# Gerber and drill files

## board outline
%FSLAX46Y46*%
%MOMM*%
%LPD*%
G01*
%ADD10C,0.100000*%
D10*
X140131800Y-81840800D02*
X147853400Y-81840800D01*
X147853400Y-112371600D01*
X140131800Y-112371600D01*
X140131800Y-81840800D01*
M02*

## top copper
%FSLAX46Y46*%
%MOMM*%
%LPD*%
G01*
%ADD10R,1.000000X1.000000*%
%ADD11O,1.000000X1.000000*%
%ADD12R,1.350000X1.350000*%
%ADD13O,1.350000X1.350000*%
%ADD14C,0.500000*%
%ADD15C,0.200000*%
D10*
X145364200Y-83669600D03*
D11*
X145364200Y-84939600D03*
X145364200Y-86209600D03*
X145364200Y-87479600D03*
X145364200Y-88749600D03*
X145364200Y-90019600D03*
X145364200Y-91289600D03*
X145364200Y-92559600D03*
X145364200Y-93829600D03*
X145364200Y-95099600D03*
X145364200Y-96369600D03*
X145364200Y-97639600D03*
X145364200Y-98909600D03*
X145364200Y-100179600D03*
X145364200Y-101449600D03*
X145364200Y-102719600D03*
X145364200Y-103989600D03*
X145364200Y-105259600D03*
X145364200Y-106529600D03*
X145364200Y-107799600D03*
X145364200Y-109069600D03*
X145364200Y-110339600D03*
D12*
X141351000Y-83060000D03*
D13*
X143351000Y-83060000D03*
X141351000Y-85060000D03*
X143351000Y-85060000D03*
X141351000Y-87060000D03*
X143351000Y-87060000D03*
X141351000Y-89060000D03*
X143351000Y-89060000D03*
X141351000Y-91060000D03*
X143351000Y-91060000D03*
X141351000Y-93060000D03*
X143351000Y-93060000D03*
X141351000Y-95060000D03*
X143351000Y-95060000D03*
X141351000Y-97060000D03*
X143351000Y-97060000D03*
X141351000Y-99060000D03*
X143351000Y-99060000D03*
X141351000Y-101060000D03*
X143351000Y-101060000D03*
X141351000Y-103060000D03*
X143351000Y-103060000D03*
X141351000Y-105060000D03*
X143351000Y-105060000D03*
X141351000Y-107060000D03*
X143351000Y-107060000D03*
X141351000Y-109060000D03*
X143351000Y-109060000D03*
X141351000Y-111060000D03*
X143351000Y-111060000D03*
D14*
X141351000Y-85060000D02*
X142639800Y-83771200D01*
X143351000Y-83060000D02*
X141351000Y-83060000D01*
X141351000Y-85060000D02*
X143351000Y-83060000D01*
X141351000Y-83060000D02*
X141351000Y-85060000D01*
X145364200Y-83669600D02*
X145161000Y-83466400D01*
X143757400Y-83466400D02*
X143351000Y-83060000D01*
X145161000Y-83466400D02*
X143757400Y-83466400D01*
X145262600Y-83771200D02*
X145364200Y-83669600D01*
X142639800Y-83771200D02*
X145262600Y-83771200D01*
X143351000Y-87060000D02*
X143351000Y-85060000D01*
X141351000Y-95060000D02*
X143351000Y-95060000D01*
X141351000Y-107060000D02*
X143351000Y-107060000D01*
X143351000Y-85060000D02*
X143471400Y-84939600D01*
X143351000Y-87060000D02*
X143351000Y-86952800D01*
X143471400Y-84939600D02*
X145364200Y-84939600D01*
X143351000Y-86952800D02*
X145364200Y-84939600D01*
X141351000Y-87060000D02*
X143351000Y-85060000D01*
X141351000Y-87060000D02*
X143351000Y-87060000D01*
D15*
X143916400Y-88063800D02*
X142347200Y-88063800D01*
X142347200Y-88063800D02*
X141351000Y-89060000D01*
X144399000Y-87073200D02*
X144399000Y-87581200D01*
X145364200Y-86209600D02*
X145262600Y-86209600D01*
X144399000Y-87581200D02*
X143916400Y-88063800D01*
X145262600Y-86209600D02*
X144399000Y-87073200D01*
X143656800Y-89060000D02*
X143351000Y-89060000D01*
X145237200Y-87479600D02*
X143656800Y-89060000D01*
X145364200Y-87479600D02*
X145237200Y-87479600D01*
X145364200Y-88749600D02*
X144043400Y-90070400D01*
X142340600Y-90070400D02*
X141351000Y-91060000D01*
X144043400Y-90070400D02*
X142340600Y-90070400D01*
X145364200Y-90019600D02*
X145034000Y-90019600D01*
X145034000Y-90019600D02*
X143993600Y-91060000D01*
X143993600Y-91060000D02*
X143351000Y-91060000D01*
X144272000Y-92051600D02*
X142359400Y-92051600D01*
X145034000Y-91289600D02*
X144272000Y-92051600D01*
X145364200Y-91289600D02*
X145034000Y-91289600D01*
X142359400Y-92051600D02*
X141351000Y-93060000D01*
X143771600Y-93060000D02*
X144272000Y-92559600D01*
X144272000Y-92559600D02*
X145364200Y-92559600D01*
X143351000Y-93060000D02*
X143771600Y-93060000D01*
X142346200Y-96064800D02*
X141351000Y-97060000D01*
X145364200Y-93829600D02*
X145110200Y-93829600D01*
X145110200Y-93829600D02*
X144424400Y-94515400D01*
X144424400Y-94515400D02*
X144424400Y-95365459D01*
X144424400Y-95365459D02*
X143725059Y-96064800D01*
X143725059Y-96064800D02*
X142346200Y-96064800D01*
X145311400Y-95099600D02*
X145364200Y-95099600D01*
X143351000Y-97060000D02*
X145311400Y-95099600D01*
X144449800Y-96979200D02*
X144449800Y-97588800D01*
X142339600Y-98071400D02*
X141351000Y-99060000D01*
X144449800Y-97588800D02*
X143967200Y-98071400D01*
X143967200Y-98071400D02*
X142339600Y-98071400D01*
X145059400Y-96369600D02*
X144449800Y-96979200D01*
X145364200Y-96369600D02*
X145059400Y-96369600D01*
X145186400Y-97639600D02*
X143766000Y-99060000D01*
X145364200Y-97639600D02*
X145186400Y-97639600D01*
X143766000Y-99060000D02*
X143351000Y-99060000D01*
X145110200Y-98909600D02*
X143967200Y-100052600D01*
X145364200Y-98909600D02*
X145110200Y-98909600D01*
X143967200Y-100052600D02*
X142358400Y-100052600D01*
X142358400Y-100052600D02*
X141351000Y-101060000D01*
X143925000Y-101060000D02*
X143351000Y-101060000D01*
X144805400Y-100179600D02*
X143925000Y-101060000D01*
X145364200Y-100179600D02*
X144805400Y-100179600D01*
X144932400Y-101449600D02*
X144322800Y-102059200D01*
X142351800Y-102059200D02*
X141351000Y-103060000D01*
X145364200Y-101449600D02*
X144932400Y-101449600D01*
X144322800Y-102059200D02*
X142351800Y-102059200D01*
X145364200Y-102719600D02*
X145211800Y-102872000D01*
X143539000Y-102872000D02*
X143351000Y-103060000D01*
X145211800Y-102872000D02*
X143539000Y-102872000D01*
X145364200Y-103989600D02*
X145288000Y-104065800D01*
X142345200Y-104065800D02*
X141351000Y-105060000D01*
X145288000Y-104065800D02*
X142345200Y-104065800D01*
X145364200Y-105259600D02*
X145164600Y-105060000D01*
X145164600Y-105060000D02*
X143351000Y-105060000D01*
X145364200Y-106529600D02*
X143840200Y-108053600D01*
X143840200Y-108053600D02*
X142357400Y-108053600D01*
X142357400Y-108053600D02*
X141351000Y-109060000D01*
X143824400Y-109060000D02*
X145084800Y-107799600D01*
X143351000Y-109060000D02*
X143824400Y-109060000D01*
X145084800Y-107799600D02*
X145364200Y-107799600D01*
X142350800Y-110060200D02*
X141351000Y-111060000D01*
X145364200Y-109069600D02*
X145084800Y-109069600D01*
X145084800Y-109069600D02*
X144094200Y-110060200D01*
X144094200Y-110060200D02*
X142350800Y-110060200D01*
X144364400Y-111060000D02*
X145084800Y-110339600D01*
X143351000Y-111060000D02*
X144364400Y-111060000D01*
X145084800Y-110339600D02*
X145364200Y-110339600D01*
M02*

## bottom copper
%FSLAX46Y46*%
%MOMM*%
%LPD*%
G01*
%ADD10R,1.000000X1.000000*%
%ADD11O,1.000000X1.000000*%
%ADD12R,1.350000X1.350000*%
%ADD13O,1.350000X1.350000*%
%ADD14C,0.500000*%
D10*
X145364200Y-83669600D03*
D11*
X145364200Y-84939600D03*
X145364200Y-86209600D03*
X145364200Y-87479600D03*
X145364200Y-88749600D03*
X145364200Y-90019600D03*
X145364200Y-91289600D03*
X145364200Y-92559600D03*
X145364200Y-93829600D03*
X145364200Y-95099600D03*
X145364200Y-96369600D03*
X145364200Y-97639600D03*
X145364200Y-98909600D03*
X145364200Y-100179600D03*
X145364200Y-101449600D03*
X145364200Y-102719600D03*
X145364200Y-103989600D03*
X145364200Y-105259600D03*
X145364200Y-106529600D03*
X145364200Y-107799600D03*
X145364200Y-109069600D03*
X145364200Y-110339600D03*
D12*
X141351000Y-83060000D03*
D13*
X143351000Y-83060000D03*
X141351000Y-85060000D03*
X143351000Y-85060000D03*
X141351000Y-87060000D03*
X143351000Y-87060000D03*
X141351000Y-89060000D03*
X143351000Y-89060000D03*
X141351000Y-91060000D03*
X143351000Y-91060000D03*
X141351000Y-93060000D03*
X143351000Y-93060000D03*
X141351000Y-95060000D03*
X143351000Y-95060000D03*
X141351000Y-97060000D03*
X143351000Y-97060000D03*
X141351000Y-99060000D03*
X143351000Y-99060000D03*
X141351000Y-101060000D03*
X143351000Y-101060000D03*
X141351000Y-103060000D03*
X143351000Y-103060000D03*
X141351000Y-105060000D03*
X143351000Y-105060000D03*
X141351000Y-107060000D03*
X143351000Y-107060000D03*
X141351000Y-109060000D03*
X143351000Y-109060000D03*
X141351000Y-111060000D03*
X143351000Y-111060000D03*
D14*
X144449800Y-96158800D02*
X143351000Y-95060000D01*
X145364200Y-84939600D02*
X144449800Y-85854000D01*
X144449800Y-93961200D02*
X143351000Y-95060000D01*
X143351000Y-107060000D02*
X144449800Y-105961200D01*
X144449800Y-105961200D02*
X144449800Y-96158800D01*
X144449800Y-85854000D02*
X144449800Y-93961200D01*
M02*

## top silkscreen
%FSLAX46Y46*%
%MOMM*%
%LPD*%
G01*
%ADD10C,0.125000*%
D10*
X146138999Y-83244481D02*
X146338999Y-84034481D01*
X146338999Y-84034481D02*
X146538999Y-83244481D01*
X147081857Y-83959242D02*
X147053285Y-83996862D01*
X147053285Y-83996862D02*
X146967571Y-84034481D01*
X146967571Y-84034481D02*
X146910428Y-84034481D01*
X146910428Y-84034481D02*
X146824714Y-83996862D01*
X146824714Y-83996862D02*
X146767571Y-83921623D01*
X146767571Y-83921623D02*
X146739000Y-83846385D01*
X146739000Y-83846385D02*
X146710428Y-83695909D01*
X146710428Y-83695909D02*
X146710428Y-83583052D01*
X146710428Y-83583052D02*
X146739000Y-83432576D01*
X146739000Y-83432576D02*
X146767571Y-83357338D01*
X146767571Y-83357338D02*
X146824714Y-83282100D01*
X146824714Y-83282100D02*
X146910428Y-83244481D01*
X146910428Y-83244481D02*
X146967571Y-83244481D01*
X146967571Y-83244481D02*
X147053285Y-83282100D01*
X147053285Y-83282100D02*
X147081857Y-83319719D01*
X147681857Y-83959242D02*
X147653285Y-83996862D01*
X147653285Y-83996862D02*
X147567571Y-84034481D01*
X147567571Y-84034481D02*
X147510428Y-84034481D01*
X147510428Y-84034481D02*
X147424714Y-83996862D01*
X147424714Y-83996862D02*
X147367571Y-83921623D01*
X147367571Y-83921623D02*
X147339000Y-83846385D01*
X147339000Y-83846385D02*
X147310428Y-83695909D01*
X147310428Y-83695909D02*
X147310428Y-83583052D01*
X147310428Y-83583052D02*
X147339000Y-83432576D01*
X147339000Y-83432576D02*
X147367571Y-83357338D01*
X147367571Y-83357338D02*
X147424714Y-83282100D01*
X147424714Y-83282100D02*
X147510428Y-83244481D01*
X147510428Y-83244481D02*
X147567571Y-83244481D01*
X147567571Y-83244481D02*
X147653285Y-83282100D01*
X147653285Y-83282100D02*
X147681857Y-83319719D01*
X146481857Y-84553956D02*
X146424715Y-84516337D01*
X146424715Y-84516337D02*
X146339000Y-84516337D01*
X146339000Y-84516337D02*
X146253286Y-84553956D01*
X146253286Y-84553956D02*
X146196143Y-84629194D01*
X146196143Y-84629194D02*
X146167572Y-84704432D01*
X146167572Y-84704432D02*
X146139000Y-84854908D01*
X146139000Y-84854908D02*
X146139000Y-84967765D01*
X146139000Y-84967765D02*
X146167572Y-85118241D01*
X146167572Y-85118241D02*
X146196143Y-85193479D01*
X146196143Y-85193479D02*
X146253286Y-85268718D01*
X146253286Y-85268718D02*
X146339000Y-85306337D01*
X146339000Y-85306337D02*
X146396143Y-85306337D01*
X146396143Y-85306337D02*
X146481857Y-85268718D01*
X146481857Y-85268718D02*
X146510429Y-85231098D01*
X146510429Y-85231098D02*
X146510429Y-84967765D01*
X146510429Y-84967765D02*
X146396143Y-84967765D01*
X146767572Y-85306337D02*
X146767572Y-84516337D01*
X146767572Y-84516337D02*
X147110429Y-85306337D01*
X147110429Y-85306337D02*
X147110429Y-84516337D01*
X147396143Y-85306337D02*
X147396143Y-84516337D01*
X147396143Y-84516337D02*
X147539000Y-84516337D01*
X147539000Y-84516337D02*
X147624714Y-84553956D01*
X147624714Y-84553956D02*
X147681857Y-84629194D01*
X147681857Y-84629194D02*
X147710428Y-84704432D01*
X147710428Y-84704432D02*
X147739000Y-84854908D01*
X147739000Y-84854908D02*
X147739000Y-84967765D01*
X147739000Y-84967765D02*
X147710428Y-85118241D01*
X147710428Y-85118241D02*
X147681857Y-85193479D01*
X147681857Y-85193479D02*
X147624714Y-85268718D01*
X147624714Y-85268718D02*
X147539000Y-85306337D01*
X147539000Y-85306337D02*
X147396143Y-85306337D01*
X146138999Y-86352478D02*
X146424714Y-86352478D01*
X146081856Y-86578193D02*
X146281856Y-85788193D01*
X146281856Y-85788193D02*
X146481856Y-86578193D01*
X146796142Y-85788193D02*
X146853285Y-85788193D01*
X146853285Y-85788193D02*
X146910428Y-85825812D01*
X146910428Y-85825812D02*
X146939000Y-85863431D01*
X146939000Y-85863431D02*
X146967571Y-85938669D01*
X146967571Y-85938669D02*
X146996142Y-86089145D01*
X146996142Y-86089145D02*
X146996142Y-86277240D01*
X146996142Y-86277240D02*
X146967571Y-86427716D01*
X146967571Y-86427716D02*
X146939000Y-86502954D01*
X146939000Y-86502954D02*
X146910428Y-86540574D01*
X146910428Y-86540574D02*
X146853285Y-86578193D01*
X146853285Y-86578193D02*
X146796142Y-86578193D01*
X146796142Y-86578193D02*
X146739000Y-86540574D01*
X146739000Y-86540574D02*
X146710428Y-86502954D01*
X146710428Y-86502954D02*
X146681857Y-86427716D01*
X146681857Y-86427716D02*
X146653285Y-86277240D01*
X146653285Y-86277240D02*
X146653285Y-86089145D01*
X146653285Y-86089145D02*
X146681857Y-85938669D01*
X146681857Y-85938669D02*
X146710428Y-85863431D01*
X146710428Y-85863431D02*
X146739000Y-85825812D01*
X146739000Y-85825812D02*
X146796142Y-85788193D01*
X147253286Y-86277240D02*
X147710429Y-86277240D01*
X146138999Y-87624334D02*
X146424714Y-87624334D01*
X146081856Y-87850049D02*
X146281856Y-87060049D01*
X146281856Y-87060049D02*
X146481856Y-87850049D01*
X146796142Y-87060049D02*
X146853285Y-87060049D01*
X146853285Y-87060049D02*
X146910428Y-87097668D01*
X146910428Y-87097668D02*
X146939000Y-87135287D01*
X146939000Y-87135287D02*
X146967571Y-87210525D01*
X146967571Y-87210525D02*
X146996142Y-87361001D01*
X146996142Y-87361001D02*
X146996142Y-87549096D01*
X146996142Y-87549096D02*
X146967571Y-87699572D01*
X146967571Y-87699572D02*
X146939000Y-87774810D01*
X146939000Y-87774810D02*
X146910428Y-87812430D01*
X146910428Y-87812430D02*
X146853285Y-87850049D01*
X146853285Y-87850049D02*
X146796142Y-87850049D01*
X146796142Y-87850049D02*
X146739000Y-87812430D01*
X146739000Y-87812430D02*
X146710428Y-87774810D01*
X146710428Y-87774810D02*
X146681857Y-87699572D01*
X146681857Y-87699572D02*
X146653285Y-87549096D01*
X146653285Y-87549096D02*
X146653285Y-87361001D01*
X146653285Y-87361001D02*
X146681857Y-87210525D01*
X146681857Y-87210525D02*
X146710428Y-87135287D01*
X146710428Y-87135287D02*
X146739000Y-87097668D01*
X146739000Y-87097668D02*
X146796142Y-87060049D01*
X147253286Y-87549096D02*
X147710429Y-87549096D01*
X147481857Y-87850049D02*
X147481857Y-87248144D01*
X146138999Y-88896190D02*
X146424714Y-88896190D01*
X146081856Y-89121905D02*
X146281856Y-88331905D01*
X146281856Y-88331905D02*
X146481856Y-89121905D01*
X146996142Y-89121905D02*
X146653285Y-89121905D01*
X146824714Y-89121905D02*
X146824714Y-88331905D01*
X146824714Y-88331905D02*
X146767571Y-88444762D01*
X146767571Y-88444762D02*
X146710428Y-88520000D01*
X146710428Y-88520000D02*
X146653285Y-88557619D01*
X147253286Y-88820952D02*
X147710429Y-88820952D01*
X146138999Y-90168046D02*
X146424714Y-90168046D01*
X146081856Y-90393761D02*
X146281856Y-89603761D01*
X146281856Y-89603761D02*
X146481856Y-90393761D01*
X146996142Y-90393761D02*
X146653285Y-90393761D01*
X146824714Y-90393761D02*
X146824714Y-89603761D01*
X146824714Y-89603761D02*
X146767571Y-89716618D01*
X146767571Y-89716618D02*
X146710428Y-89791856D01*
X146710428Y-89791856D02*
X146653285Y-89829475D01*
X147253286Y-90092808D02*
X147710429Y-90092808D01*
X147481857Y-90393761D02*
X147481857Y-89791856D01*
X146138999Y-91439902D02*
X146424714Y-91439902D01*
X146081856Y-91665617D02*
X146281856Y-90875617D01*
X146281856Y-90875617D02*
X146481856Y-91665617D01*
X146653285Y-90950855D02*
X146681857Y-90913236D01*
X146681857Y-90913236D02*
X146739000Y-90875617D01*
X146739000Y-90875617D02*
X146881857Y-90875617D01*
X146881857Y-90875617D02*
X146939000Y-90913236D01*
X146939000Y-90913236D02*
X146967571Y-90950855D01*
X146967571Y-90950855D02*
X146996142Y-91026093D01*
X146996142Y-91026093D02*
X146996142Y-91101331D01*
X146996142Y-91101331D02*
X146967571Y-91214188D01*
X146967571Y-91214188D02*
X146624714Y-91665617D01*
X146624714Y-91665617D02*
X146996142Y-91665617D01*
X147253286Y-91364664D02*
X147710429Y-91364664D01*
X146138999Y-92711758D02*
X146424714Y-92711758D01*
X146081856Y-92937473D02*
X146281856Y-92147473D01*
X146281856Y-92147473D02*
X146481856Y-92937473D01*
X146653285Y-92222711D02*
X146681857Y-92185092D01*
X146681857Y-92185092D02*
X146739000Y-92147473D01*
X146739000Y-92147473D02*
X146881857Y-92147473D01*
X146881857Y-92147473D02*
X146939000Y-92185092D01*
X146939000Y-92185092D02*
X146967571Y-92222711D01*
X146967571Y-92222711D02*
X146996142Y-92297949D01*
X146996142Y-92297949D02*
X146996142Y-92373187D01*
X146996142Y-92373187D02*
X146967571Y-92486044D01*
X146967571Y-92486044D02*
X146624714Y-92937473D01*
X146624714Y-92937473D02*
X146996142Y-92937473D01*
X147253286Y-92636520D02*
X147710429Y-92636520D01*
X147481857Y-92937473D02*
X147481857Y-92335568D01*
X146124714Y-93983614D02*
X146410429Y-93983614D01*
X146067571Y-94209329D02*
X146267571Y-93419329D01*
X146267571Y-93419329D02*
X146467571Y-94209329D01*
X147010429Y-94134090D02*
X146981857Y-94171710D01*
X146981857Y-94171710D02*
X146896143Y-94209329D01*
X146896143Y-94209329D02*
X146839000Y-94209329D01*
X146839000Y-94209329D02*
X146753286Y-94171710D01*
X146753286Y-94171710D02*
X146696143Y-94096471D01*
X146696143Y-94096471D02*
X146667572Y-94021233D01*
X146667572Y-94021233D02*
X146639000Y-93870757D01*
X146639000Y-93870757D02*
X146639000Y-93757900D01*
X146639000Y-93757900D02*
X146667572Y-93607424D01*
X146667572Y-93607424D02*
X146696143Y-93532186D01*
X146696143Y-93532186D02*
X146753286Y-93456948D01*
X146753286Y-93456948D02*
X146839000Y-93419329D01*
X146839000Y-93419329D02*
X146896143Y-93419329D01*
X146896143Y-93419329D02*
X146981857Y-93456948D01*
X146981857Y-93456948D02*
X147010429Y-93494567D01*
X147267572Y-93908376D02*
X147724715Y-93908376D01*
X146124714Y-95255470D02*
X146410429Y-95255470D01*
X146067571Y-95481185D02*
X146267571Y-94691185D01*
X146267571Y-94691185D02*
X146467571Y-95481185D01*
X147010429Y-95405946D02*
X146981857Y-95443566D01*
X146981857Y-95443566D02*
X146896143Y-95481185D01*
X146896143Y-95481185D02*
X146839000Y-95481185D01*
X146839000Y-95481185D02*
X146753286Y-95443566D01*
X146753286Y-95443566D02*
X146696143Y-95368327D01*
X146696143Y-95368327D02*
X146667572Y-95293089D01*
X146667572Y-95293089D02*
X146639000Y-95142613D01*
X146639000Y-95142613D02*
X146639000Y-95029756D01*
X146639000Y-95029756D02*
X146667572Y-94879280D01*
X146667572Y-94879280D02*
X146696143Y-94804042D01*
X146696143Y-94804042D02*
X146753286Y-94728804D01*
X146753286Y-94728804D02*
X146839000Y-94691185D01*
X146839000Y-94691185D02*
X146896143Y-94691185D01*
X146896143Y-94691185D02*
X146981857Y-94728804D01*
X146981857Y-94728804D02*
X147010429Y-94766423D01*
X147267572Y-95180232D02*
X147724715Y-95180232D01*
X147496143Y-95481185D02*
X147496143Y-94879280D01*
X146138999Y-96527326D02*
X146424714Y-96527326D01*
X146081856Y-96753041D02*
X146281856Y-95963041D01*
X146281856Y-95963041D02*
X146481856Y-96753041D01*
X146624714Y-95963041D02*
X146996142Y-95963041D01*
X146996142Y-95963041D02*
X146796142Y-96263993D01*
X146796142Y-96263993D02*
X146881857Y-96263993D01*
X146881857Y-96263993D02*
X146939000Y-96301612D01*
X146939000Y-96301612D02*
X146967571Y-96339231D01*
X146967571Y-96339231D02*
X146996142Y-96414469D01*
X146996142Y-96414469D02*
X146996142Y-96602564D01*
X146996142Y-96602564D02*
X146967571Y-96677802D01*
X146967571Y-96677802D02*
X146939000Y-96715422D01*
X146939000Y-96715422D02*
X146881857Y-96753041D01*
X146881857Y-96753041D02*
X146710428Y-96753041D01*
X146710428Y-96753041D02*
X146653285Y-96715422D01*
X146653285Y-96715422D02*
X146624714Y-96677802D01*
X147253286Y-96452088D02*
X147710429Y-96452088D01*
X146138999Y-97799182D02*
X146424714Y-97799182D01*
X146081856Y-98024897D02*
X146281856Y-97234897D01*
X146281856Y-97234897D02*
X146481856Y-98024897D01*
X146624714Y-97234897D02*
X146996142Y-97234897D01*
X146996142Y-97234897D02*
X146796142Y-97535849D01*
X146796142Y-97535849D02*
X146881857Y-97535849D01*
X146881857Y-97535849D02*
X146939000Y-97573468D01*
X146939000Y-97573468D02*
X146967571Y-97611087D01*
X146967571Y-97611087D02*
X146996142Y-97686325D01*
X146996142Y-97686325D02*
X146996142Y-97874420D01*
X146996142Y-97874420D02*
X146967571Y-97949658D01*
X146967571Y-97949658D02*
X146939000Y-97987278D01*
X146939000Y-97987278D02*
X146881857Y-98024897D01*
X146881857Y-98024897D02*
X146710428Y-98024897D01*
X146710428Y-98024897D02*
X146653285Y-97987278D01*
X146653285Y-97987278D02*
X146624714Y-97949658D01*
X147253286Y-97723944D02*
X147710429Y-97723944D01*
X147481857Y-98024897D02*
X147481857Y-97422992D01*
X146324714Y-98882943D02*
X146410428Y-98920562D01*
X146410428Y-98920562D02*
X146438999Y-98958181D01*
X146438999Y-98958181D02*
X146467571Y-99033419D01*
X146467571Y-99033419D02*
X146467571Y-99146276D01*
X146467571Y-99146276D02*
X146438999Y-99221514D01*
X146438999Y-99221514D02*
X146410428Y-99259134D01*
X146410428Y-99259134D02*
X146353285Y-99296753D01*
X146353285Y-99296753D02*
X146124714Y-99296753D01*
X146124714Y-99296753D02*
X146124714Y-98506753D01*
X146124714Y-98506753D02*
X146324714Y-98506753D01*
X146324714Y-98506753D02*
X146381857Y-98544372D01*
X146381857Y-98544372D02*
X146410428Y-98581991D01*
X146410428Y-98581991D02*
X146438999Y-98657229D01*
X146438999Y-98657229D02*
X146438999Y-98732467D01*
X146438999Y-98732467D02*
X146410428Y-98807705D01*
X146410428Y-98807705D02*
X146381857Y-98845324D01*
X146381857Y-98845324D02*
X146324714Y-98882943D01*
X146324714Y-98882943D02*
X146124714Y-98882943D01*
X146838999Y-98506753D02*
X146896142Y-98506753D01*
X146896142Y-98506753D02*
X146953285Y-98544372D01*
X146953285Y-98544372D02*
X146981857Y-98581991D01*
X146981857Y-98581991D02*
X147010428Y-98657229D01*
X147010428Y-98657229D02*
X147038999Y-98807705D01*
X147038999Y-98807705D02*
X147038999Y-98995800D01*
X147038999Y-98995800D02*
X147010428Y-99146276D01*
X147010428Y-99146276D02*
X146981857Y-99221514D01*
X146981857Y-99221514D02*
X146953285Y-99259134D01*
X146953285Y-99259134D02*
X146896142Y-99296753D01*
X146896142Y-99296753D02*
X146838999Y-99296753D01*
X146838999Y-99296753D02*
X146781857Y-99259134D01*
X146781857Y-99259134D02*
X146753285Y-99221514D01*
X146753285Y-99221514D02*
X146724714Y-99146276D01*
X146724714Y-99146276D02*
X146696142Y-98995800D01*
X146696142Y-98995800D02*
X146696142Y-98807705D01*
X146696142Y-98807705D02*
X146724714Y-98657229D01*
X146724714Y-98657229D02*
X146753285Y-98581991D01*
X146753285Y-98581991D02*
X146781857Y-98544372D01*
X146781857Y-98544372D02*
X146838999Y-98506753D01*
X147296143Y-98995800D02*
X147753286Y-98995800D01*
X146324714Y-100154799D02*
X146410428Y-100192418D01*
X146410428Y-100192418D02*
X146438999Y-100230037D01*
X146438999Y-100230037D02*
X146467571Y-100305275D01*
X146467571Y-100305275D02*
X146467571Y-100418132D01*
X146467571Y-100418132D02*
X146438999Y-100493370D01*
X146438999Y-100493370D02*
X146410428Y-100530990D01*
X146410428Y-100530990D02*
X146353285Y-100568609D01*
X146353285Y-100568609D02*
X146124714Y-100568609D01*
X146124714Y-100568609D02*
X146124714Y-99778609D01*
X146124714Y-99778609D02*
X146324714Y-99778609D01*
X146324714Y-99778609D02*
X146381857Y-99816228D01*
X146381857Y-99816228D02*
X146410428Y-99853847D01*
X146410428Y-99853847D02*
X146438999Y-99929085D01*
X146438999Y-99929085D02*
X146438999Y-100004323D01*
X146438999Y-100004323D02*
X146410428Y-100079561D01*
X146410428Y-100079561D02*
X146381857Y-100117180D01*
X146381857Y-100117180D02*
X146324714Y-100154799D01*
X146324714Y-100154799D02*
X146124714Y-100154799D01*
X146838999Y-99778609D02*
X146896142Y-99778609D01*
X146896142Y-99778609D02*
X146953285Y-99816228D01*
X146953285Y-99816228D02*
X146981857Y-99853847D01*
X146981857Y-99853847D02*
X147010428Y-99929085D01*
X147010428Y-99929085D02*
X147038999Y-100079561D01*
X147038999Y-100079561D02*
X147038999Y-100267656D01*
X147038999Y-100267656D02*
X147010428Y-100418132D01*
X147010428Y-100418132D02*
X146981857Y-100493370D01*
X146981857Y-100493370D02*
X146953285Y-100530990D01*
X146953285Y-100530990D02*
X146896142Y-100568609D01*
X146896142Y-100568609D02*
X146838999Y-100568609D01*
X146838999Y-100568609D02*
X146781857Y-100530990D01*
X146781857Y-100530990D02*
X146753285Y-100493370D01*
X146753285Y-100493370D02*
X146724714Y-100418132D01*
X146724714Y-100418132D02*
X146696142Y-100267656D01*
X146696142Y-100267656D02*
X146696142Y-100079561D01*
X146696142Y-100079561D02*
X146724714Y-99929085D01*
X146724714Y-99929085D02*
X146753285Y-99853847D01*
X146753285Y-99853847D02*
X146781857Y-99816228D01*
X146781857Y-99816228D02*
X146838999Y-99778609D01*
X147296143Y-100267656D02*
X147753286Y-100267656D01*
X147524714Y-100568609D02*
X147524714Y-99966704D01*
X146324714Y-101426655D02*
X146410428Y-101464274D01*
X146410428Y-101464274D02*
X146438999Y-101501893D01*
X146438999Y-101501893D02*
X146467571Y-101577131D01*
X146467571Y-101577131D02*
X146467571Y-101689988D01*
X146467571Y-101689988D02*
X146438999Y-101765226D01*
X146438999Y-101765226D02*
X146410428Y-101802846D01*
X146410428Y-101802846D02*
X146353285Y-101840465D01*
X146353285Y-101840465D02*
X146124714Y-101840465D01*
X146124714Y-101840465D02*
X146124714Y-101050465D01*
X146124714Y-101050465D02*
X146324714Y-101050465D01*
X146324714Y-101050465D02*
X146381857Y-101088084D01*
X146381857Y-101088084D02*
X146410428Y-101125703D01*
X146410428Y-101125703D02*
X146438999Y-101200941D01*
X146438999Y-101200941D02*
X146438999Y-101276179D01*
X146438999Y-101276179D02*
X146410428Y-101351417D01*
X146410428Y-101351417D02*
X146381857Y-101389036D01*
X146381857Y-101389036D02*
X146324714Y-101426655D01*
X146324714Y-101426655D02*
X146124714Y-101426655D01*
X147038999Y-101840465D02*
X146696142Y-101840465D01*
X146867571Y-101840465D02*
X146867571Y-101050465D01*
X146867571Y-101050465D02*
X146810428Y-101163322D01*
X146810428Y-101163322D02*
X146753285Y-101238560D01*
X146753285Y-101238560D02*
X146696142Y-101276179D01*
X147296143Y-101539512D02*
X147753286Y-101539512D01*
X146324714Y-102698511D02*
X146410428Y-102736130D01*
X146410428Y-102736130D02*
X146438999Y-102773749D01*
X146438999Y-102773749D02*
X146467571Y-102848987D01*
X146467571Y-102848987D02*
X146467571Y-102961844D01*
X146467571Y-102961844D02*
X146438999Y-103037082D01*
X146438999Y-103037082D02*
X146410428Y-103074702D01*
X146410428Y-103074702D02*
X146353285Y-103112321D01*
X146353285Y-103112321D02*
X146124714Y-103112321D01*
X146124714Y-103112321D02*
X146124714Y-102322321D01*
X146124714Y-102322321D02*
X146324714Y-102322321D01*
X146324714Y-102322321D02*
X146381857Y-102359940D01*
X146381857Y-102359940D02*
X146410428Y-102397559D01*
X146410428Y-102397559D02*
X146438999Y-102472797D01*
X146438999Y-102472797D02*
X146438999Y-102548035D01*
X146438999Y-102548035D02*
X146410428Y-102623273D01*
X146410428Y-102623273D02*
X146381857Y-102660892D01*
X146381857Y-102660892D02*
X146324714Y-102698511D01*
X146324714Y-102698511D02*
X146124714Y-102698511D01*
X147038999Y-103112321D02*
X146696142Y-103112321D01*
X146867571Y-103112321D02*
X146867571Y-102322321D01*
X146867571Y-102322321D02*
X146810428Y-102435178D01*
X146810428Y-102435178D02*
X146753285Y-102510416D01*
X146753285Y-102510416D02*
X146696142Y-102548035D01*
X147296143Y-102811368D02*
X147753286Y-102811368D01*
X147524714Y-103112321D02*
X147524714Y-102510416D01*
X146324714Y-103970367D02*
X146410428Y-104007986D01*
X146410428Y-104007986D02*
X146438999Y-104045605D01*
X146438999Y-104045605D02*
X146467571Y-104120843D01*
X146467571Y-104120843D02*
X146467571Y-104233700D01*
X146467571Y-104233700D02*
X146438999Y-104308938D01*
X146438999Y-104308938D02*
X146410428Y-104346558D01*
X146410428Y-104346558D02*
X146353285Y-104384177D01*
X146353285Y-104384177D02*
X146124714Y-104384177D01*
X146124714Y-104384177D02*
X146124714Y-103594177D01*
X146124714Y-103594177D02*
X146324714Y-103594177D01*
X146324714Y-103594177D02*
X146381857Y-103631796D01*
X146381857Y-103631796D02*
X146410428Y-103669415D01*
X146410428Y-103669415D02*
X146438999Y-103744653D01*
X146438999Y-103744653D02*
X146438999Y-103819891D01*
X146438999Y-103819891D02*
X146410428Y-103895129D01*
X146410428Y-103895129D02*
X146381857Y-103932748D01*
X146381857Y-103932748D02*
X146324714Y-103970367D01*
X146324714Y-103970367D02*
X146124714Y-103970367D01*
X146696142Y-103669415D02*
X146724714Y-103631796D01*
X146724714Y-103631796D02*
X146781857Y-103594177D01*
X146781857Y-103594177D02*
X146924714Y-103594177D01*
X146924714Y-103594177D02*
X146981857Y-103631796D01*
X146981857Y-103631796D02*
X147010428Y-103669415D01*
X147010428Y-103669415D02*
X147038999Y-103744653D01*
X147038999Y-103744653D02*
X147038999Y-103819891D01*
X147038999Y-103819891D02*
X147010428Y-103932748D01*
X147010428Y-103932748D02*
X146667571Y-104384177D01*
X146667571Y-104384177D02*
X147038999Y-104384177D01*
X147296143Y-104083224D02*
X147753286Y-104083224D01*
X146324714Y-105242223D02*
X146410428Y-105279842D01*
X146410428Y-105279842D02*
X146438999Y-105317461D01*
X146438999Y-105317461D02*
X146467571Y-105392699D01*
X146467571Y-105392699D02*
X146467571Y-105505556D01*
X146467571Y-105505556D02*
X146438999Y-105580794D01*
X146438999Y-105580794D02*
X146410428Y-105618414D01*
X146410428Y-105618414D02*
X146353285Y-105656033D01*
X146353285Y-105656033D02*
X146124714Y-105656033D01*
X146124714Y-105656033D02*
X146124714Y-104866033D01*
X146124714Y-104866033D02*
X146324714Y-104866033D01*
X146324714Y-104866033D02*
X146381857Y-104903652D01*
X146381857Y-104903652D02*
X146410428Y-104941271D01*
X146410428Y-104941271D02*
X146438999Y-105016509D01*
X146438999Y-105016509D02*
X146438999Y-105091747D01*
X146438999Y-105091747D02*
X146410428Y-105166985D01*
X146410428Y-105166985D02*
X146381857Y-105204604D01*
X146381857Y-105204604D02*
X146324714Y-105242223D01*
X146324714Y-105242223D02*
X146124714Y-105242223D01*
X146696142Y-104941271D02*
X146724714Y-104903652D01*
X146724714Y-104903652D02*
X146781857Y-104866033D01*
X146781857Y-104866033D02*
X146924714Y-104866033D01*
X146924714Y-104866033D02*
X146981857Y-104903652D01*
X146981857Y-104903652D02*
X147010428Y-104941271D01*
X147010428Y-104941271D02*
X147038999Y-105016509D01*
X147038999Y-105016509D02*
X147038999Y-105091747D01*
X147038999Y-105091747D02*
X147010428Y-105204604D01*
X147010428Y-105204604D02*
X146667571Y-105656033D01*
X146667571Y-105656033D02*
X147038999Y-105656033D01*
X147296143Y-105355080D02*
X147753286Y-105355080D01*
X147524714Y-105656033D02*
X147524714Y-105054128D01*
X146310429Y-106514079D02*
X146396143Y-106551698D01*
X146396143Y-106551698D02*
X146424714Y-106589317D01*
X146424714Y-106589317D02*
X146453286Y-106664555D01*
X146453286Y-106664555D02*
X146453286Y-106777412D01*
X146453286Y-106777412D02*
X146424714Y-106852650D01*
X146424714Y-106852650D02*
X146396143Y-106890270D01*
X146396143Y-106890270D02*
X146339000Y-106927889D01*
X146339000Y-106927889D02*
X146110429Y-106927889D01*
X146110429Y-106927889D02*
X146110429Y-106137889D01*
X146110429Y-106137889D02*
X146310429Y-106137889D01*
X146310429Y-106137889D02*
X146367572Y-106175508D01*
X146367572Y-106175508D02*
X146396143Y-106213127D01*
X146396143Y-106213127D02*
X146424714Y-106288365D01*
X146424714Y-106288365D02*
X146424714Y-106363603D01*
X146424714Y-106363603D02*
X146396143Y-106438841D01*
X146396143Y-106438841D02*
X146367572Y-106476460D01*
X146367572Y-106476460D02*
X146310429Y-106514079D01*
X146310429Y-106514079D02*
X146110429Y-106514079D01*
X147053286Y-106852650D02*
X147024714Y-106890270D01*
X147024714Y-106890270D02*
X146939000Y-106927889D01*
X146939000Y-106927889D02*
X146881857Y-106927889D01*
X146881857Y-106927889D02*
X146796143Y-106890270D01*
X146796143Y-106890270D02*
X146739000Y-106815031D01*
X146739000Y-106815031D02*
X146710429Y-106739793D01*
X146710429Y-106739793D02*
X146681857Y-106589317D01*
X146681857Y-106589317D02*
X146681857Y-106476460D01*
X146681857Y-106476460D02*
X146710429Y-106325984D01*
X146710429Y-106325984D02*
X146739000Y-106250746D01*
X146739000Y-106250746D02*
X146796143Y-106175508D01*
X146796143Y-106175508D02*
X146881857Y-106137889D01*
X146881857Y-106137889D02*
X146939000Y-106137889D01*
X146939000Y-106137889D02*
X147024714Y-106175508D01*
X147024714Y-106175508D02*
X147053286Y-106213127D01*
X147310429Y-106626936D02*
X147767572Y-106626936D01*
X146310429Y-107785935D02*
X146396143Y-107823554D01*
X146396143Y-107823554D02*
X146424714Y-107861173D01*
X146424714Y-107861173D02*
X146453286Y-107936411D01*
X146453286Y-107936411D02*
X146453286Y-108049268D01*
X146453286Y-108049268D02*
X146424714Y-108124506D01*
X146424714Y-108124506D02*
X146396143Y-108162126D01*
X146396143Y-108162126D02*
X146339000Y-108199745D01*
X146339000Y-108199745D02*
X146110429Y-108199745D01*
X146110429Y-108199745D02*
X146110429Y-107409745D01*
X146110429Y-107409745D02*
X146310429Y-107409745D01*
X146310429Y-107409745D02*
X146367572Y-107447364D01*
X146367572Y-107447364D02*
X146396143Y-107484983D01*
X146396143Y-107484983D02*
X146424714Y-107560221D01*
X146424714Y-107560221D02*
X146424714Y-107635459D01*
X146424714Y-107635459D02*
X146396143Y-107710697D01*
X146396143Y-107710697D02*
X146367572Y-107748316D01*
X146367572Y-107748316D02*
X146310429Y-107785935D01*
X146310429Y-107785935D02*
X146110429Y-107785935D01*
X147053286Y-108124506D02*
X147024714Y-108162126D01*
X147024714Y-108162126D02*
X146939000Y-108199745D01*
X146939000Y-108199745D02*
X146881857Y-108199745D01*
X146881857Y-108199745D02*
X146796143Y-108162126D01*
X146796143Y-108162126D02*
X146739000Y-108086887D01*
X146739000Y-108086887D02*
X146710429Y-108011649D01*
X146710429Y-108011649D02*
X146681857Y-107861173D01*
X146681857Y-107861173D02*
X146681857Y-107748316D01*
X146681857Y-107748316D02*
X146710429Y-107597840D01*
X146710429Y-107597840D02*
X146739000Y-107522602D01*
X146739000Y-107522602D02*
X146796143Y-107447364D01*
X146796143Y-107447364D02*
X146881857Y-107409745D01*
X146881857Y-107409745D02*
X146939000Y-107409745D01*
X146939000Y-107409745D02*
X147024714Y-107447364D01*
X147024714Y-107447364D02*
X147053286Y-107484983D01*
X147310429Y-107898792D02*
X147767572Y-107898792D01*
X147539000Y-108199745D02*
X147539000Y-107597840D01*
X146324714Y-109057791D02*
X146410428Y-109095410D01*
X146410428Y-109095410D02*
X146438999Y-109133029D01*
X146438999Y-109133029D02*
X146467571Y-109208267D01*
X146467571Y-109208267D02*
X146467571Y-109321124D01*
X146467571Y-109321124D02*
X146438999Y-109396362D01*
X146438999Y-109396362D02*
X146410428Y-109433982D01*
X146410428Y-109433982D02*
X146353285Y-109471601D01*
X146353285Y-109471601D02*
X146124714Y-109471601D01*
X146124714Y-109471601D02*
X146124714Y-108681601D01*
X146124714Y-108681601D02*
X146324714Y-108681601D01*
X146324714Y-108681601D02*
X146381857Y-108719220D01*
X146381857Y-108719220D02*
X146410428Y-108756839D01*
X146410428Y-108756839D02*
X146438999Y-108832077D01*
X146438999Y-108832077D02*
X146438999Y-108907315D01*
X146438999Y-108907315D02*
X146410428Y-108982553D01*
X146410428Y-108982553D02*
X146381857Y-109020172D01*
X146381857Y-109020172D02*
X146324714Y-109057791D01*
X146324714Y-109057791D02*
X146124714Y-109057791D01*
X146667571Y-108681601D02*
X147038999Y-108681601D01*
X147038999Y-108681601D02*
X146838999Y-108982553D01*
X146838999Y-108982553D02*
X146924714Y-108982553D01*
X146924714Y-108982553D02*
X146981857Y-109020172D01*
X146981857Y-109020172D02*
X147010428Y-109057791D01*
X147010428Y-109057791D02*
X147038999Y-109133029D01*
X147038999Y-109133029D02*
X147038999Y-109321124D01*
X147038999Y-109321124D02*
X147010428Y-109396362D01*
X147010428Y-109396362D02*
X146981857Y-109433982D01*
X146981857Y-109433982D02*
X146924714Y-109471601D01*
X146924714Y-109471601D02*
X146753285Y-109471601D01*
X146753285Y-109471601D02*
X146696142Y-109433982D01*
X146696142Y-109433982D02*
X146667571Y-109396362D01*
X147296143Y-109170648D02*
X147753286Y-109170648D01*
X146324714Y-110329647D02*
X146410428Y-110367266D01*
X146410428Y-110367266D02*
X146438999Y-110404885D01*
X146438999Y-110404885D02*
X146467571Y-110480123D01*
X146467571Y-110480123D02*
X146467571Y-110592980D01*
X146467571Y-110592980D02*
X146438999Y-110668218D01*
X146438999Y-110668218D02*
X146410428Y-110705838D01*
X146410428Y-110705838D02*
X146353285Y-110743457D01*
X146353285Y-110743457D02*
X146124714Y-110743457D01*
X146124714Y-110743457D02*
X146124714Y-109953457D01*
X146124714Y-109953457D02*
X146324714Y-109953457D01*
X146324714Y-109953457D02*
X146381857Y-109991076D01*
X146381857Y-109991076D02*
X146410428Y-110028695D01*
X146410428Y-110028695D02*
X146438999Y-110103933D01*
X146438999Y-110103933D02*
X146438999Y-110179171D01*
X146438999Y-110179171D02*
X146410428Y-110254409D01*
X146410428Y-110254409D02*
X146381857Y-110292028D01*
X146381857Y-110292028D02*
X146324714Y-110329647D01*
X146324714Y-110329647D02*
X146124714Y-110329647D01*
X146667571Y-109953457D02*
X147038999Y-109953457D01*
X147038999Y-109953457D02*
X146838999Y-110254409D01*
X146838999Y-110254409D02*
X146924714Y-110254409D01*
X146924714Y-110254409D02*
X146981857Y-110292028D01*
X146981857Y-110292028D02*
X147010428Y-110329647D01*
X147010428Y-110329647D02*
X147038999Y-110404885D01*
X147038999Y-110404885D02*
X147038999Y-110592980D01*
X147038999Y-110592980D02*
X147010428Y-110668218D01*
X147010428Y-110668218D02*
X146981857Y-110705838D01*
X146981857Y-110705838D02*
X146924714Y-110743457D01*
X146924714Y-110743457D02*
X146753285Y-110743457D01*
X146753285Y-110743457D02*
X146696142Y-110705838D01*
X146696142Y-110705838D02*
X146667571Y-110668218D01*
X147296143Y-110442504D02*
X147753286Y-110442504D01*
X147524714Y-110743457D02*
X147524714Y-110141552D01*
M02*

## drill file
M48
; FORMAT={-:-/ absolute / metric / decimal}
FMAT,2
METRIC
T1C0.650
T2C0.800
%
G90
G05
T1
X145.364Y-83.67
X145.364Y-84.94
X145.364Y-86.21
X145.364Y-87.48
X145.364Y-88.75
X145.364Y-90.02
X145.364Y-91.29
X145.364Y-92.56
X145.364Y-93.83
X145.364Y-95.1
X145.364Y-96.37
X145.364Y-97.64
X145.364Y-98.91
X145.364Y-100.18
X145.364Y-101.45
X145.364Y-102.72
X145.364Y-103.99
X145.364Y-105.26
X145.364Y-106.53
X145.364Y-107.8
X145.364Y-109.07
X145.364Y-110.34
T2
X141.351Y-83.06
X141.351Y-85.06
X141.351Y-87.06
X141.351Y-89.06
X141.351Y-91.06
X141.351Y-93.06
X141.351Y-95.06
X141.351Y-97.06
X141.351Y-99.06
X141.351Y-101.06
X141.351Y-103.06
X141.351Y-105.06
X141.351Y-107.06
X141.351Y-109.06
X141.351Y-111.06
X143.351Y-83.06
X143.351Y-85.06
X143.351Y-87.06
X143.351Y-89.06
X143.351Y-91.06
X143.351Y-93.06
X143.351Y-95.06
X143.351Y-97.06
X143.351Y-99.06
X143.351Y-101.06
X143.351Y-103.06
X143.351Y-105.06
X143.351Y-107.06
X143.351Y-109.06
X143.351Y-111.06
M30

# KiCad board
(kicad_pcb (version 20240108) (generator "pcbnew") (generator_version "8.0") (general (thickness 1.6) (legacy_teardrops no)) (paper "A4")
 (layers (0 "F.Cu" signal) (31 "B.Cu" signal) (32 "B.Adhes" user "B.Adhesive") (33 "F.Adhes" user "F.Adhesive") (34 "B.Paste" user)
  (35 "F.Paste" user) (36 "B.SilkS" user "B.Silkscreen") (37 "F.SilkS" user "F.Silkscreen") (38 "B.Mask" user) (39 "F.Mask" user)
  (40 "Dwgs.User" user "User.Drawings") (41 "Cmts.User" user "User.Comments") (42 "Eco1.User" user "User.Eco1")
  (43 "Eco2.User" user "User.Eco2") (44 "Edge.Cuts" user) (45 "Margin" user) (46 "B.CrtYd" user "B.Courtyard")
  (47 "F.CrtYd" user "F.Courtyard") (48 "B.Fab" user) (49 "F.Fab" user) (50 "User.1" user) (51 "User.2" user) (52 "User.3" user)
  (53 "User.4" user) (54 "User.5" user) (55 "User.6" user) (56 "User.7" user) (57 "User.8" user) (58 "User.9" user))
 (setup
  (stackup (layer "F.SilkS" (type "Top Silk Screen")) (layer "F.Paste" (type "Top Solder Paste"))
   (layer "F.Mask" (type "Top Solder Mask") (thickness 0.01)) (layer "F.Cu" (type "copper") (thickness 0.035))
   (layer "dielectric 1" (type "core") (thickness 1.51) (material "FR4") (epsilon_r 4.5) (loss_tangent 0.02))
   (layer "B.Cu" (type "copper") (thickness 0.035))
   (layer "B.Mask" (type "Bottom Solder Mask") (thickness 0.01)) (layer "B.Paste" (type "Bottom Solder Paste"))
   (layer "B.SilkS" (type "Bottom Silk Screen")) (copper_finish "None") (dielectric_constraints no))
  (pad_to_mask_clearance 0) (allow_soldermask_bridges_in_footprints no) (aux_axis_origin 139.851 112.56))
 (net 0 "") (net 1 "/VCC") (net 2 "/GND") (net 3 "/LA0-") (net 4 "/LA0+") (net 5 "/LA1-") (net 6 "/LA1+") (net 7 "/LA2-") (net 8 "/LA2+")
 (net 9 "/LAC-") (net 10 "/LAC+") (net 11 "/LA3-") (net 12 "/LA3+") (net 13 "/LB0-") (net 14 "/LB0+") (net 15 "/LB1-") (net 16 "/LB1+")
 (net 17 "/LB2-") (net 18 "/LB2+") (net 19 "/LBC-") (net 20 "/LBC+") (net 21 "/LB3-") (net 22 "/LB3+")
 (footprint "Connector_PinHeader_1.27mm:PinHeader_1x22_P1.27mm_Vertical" (layer "B.Cu") (at 145.3642 83.6696 180)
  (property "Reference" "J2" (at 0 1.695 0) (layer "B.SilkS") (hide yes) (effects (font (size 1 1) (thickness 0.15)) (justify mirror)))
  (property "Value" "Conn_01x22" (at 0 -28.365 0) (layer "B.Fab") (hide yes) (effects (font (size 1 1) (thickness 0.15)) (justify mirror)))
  (pad "1" thru_hole rect (at 0 0 180) (size 1 1) (drill 0.65) (layers "*.Cu" "*.Mask") (remove_unused_layers no) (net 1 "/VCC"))
  (pad "2" thru_hole oval (at 0 -1.27 180) (size 1 1) (drill 0.65) (layers "*.Cu" "*.Mask") (remove_unused_layers no) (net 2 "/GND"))
  (pad "3" thru_hole oval (at 0 -2.54 180) (size 1 1) (drill 0.65) (layers "*.Cu" "*.Mask") (remove_unused_layers no) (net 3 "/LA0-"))
  (pad "4" thru_hole oval (at 0 -3.81 180) (size 1 1) (drill 0.65) (layers "*.Cu" "*.Mask") (remove_unused_layers no) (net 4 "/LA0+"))
  (pad "5" thru_hole oval (at 0 -5.08 180) (size 1 1) (drill 0.65) (layers "*.Cu" "*.Mask") (remove_unused_layers no) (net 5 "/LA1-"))
  (pad "6" thru_hole oval (at 0 -6.35 180) (size 1 1) (drill 0.65) (layers "*.Cu" "*.Mask") (remove_unused_layers no) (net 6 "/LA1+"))
  (pad "7" thru_hole oval (at 0 -7.62 180) (size 1 1) (drill 0.65) (layers "*.Cu" "*.Mask") (remove_unused_layers no) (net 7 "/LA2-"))
  (pad "8" thru_hole oval (at 0 -8.89 180) (size 1 1) (drill 0.65) (layers "*.Cu" "*.Mask") (remove_unused_layers no) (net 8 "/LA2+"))
  (pad "9" thru_hole oval (at 0 -10.16 180) (size 1 1) (drill 0.65) (layers "*.Cu" "*.Mask") (remove_unused_layers no) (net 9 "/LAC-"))
  (pad "10" thru_hole oval (at 0 -11.43 180) (size 1 1) (drill 0.65) (layers "*.Cu" "*.Mask") (remove_unused_layers no) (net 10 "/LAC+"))
  (pad "11" thru_hole oval (at 0 -12.7 180) (size 1 1) (drill 0.65) (layers "*.Cu" "*.Mask") (remove_unused_layers no) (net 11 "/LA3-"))
  (pad "12" thru_hole oval (at 0 -13.97 180) (size 1 1) (drill 0.65) (layers "*.Cu" "*.Mask") (remove_unused_layers no) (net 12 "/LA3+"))
  (pad "13" thru_hole oval (at 0 -15.24 180) (size 1 1) (drill 0.65) (layers "*.Cu" "*.Mask") (remove_unused_layers no) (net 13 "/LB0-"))
  (pad "14" thru_hole oval (at 0 -16.51 180) (size 1 1) (drill 0.65) (layers "*.Cu" "*.Mask") (remove_unused_layers no) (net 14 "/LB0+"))
  (pad "15" thru_hole oval (at 0 -17.78 180) (size 1 1) (drill 0.65) (layers "*.Cu" "*.Mask") (remove_unused_layers no) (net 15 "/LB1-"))
  (pad "16" thru_hole oval (at 0 -19.05 180) (size 1 1) (drill 0.65) (layers "*.Cu" "*.Mask") (remove_unused_layers no) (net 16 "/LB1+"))
  (pad "17" thru_hole oval (at 0 -20.32 180) (size 1 1) (drill 0.65) (layers "*.Cu" "*.Mask") (remove_unused_layers no) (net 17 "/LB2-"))
  (pad "18" thru_hole oval (at 0 -21.59 180) (size 1 1) (drill 0.65) (layers "*.Cu" "*.Mask") (remove_unused_layers no) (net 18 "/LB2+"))
  (pad "19" thru_hole oval (at 0 -22.86 180) (size 1 1) (drill 0.65) (layers "*.Cu" "*.Mask") (remove_unused_layers no) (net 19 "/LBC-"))
  (pad "20" thru_hole oval (at 0 -24.13 180) (size 1 1) (drill 0.65) (layers "*.Cu" "*.Mask") (remove_unused_layers no) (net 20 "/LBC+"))
  (pad "21" thru_hole oval (at 0 -25.4 180) (size 1 1) (drill 0.65) (layers "*.Cu" "*.Mask") (remove_unused_layers no) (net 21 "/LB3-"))
  (pad "22" thru_hole oval (at 0 -26.67 180) (size 1 1) (drill 0.65) (layers "*.Cu" "*.Mask") (remove_unused_layers no) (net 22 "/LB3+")))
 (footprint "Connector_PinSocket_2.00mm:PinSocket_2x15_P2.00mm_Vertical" (layer "B.Cu") (at 141.351 83.06 180)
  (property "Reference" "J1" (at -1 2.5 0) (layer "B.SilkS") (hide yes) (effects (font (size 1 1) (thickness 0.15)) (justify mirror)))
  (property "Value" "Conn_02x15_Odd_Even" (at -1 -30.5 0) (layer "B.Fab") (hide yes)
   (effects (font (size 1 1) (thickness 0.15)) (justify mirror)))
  (pad "1" thru_hole rect (at 0 0 180) (size 1.35 1.35) (drill 0.8) (layers "*.Cu" "*.Mask") (remove_unused_layers no) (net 1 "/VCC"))
  (pad "2" thru_hole oval (at -2 0 180) (size 1.35 1.35) (drill 0.8) (layers "*.Cu" "*.Mask") (remove_unused_layers no) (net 1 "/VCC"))
  (pad "3" thru_hole oval (at 0 -2 180) (size 1.35 1.35) (drill 0.8) (layers "*.Cu" "*.Mask") (remove_unused_layers no) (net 1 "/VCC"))
  (pad "4" thru_hole oval (at -2 -2 180) (size 1.35 1.35) (drill 0.8) (layers "*.Cu" "*.Mask") (remove_unused_layers no) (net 2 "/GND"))
  (pad "5" thru_hole oval (at 0 -4 180) (size 1.35 1.35) (drill 0.8) (layers "*.Cu" "*.Mask") (remove_unused_layers no) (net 2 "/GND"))
  (pad "6" thru_hole oval (at -2 -4 180) (size 1.35 1.35) (drill 0.8) (layers "*.Cu" "*.Mask") (remove_unused_layers no) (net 2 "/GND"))
  (pad "7" thru_hole oval (at 0 -6 180) (size 1.35 1.35) (drill 0.8) (layers "*.Cu" "*.Mask") (remove_unused_layers no) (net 3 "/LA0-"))
  (pad "8" thru_hole oval (at -2 -6 180) (size 1.35 1.35) (drill 0.8) (layers "*.Cu" "*.Mask") (remove_unused_layers no) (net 4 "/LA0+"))
  (pad "9" thru_hole oval (at 0 -8 180) (size 1.35 1.35) (drill 0.8) (layers "*.Cu" "*.Mask") (remove_unused_layers no) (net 5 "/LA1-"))
  (pad "10" thru_hole oval (at -2 -8 180) (size 1.35 1.35) (drill 0.8) (layers "*.Cu" "*.Mask") (remove_unused_layers no) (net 6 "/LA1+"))
  (pad "11" thru_hole oval (at 0 -10 180) (size 1.35 1.35) (drill 0.8) (layers "*.Cu" "*.Mask") (remove_unused_layers no) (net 7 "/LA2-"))
  (pad "12" thru_hole oval (at -2 -10 180) (size 1.35 1.35) (drill 0.8) (layers "*.Cu" "*.Mask") (remove_unused_layers no) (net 8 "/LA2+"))
  (pad "13" thru_hole oval (at 0 -12 180) (size 1.35 1.35) (drill 0.8) (layers "*.Cu" "*.Mask") (remove_unused_layers no) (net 2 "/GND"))
  (pad "14" thru_hole oval (at -2 -12 180) (size 1.35 1.35) (drill 0.8) (layers "*.Cu" "*.Mask") (remove_unused_layers no) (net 2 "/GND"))
  (pad "15" thru_hole oval (at 0 -14 180) (size 1.35 1.35) (drill 0.8) (layers "*.Cu" "*.Mask") (remove_unused_layers no) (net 9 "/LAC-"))
  (pad "16" thru_hole oval (at -2 -14 180) (size 1.35 1.35) (drill 0.8) (layers "*.Cu" "*.Mask") (remove_unused_layers no) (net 10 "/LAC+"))
  (pad "17" thru_hole oval (at 0 -16 180) (size 1.35 1.35) (drill 0.8) (layers "*.Cu" "*.Mask") (remove_unused_layers no) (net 11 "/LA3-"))
  (pad "18" thru_hole oval (at -2 -16 180) (size 1.35 1.35) (drill 0.8) (layers "*.Cu" "*.Mask") (remove_unused_layers no) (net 12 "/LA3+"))
  (pad "19" thru_hole oval (at 0 -18 180) (size 1.35 1.35) (drill 0.8) (layers "*.Cu" "*.Mask") (remove_unused_layers no) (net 13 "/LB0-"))
  (pad "20" thru_hole oval (at -2 -18 180) (size 1.35 1.35) (drill 0.8) (layers "*.Cu" "*.Mask") (remove_unused_layers no) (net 14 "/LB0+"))
  (pad "21" thru_hole oval (at 0 -20 180) (size 1.35 1.35) (drill 0.8) (layers "*.Cu" "*.Mask") (remove_unused_layers no) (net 15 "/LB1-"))
  (pad "22" thru_hole oval (at -2 -20 180) (size 1.35 1.35) (drill 0.8) (layers "*.Cu" "*.Mask") (remove_unused_layers no) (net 16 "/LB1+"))
  (pad "23" thru_hole oval (at 0 -22 180) (size 1.35 1.35) (drill 0.8) (layers "*.Cu" "*.Mask") (remove_unused_layers no) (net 17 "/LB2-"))
  (pad "24" thru_hole oval (at -2 -22 180) (size 1.35 1.35) (drill 0.8) (layers "*.Cu" "*.Mask") (remove_unused_layers no) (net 18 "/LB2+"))
  (pad "25" thru_hole oval (at 0 -24 180) (size 1.35 1.35) (drill 0.8) (layers "*.Cu" "*.Mask") (remove_unused_layers no) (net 2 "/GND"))
  (pad "26" thru_hole oval (at -2 -24 180) (size 1.35 1.35) (drill 0.8) (layers "*.Cu" "*.Mask") (remove_unused_layers no) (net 2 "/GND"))
  (pad "27" thru_hole oval (at 0 -26 180) (size 1.35 1.35) (drill 0.8) (layers "*.Cu" "*.Mask") (remove_unused_layers no) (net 19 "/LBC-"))
  (pad "28" thru_hole oval (at -2 -26 180) (size 1.35 1.35) (drill 0.8) (layers "*.Cu" "*.Mask") (remove_unused_layers no) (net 20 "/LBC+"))
  (pad "29" thru_hole oval (at 0 -28 180) (size 1.35 1.35) (drill 0.8) (layers "*.Cu" "*.Mask") (remove_unused_layers no) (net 21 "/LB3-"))
  (pad "30" thru_hole oval (at -2 -28 180) (size 1.35 1.35) (drill 0.8) (layers "*.Cu" "*.Mask") (remove_unused_layers no) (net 22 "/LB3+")))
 (gr_rect (start 140.1318 81.8408) (end 147.8534 112.3716) (stroke (width 0.1) (type solid)) (fill none) (layer "Edge.Cuts"))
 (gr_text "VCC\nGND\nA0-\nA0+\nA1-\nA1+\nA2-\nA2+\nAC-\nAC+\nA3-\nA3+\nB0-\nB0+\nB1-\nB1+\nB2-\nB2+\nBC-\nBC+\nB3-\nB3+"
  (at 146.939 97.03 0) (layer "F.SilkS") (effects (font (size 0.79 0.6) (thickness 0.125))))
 (segment (start 141.351 85.06) (end 142.6398 83.7712) (width 0.5) (layer "F.Cu") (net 1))
 (segment (start 143.351 83.06) (end 141.351 83.06) (width 0.5) (layer "F.Cu") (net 1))
 (segment (start 141.351 85.06) (end 143.351 83.06) (width 0.5) (layer "F.Cu") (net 1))
 (segment (start 141.351 83.06) (end 141.351 85.06) (width 0.5) (layer "F.Cu") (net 1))
 (segment (start 145.3642 83.6696) (end 145.161 83.4664) (width 0.5) (layer "F.Cu") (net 1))
 (segment (start 143.7574 83.4664) (end 143.351 83.06) (width 0.5) (layer "F.Cu") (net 1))
 (segment (start 145.161 83.4664) (end 143.7574 83.4664) (width 0.5) (layer "F.Cu") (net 1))
 (segment (start 145.2626 83.7712) (end 145.3642 83.6696) (width 0.5) (layer "F.Cu") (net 1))
 (segment (start 142.6398 83.7712) (end 145.2626 83.7712) (width 0.5) (layer "F.Cu") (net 1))
 (segment (start 143.351 87.06) (end 143.351 85.06) (width 0.5) (layer "F.Cu") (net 2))
 (segment (start 141.351 95.06) (end 143.351 95.06) (width 0.5) (layer "F.Cu") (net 2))
 (segment (start 141.351 107.06) (end 143.351 107.06) (width 0.5) (layer "F.Cu") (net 2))
 (segment (start 143.351 85.06) (end 143.4714 84.9396) (width 0.5) (layer "F.Cu") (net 2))
 (segment (start 143.351 87.06) (end 143.351 86.9528) (width 0.5) (layer "F.Cu") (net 2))
 (segment (start 143.4714 84.9396) (end 145.3642 84.9396) (width 0.5) (layer "F.Cu") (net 2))
 (segment (start 143.351 86.9528) (end 145.3642 84.9396) (width 0.5) (layer "F.Cu") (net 2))
 (segment (start 141.351 87.06) (end 143.351 85.06) (width 0.5) (layer "F.Cu") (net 2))
 (segment (start 141.351 87.06) (end 143.351 87.06) (width 0.5) (layer "F.Cu") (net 2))
 (segment (start 144.4498 96.1588) (end 143.351 95.06) (width 0.5) (layer "B.Cu") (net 2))
 (segment (start 145.3642 84.9396) (end 144.4498 85.854) (width 0.5) (layer "B.Cu") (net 2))
 (segment (start 144.4498 93.9612) (end 143.351 95.06) (width 0.5) (layer "B.Cu") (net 2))
 (segment (start 143.351 107.06) (end 144.4498 105.9612) (width 0.5) (layer "B.Cu") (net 2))
 (segment (start 144.4498 105.9612) (end 144.4498 96.1588) (width 0.5) (layer "B.Cu") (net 2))
 (segment (start 144.4498 85.854) (end 144.4498 93.9612) (width 0.5) (layer "B.Cu") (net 2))
 (segment (start 143.9164 88.0638) (end 142.3472 88.0638) (width 0.2) (layer "F.Cu") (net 3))
 (segment (start 142.3472 88.0638) (end 141.351 89.06) (width 0.2) (layer "F.Cu") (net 3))
 (segment (start 144.399 87.0732) (end 144.399 87.5812) (width 0.2) (layer "F.Cu") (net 3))
 (segment (start 145.3642 86.2096) (end 145.2626 86.2096) (width 0.2) (layer "F.Cu") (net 3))
 (segment (start 144.399 87.5812) (end 143.9164 88.0638) (width 0.2) (layer "F.Cu") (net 3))
 (segment (start 145.2626 86.2096) (end 144.399 87.0732) (width 0.2) (layer "F.Cu") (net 3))
 (segment (start 143.6568 89.06) (end 143.351 89.06) (width 0.2) (layer "F.Cu") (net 4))
 (segment (start 145.2372 87.4796) (end 143.6568 89.06) (width 0.2) (layer "F.Cu") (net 4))
 (segment (start 145.3642 87.4796) (end 145.2372 87.4796) (width 0.2) (layer "F.Cu") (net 4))
 (segment (start 145.3642 88.7496) (end 144.0434 90.0704) (width 0.2) (layer "F.Cu") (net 5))
 (segment (start 142.3406 90.0704) (end 141.351 91.06) (width 0.2) (layer "F.Cu") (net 5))
 (segment (start 144.0434 90.0704) (end 142.3406 90.0704) (width 0.2) (layer "F.Cu") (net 5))
 (segment (start 145.3642 90.0196) (end 145.034 90.0196) (width 0.2) (layer "F.Cu") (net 6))
 (segment (start 145.034 90.0196) (end 143.9936 91.06) (width 0.2) (layer "F.Cu") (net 6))
 (segment (start 143.9936 91.06) (end 143.351 91.06) (width 0.2) (layer "F.Cu") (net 6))
 (segment (start 144.272 92.0516) (end 142.3594 92.0516) (width 0.2) (layer "F.Cu") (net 7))
 (segment (start 145.034 91.2896) (end 144.272 92.0516) (width 0.2) (layer "F.Cu") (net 7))
 (segment (start 145.3642 91.2896) (end 145.034 91.2896) (width 0.2) (layer "F.Cu") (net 7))
 (segment (start 142.3594 92.0516) (end 141.351 93.06) (width 0.2) (layer "F.Cu") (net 7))
 (segment (start 143.7716 93.06) (end 144.272 92.5596) (width 0.2) (layer "F.Cu") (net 8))
 (segment (start 144.272 92.5596) (end 145.3642 92.5596) (width 0.2) (layer "F.Cu") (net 8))
 (segment (start 143.351 93.06) (end 143.7716 93.06) (width 0.2) (layer "F.Cu") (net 8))
 (segment (start 142.3462 96.0648) (end 141.351 97.06) (width 0.2) (layer "F.Cu") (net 9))
 (segment (start 145.3642 93.8296) (end 145.1102 93.8296) (width 0.2) (layer "F.Cu") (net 9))
 (segment (start 145.1102 93.8296) (end 144.4244 94.5154) (width 0.2) (layer "F.Cu") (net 9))
 (segment (start 144.4244 94.5154) (end 144.4244 95.365459) (width 0.2) (layer "F.Cu") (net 9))
 (segment (start 144.4244 95.365459) (end 143.725059 96.0648) (width 0.2) (layer "F.Cu") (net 9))
 (segment (start 143.725059 96.0648) (end 142.3462 96.0648) (width 0.2) (layer "F.Cu") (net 9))
 (segment (start 145.3114 95.0996) (end 145.3642 95.0996) (width 0.2) (layer "F.Cu") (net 10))
 (segment (start 143.351 97.06) (end 145.3114 95.0996) (width 0.2) (layer "F.Cu") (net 10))
 (segment (start 144.4498 96.9792) (end 144.4498 97.5888) (width 0.2) (layer "F.Cu") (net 11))
 (segment (start 142.3396 98.0714) (end 141.351 99.06) (width 0.2) (layer "F.Cu") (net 11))
 (segment (start 144.4498 97.5888) (end 143.9672 98.0714) (width 0.2) (layer "F.Cu") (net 11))
 (segment (start 143.9672 98.0714) (end 142.3396 98.0714) (width 0.2) (layer "F.Cu") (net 11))
 (segment (start 145.0594 96.3696) (end 144.4498 96.9792) (width 0.2) (layer "F.Cu") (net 11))
 (segment (start 145.3642 96.3696) (end 145.0594 96.3696) (width 0.2) (layer "F.Cu") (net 11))
 (segment (start 145.1864 97.6396) (end 143.766 99.06) (width 0.2) (layer "F.Cu") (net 12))
 (segment (start 145.3642 97.6396) (end 145.1864 97.6396) (width 0.2) (layer "F.Cu") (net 12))
 (segment (start 143.766 99.06) (end 143.351 99.06) (width 0.2) (layer "F.Cu") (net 12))
 (segment (start 145.1102 98.9096) (end 143.9672 100.0526) (width 0.2) (layer "F.Cu") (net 13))
 (segment (start 145.3642 98.9096) (end 145.1102 98.9096) (width 0.2) (layer "F.Cu") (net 13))
 (segment (start 143.9672 100.0526) (end 142.3584 100.0526) (width 0.2) (layer "F.Cu") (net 13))
 (segment (start 142.3584 100.0526) (end 141.351 101.06) (width 0.2) (layer "F.Cu") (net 13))
 (segment (start 143.925 101.06) (end 143.351 101.06) (width 0.2) (layer "F.Cu") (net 14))
 (segment (start 144.8054 100.1796) (end 143.925 101.06) (width 0.2) (layer "F.Cu") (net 14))
 (segment (start 145.3642 100.1796) (end 144.8054 100.1796) (width 0.2) (layer "F.Cu") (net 14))
 (segment (start 144.9324 101.4496) (end 144.3228 102.0592) (width 0.2) (layer "F.Cu") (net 15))
 (segment (start 142.3518 102.0592) (end 141.351 103.06) (width 0.2) (layer "F.Cu") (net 15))
 (segment (start 145.3642 101.4496) (end 144.9324 101.4496) (width 0.2) (layer "F.Cu") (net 15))
 (segment (start 144.3228 102.0592) (end 142.3518 102.0592) (width 0.2) (layer "F.Cu") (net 15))
 (segment (start 145.3642 102.7196) (end 145.2118 102.872) (width 0.2) (layer "F.Cu") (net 16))
 (segment (start 143.539 102.872) (end 143.351 103.06) (width 0.2) (layer "F.Cu") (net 16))
 (segment (start 145.2118 102.872) (end 143.539 102.872) (width 0.2) (layer "F.Cu") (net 16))
 (segment (start 145.3642 103.9896) (end 145.288 104.0658) (width 0.2) (layer "F.Cu") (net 17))
 (segment (start 142.3452 104.0658) (end 141.351 105.06) (width 0.2) (layer "F.Cu") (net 17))
 (segment (start 145.288 104.0658) (end 142.3452 104.0658) (width 0.2) (layer "F.Cu") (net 17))
 (segment (start 145.3642 105.2596) (end 145.1646 105.06) (width 0.2) (layer "F.Cu") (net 18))
 (segment (start 145.1646 105.06) (end 143.351 105.06) (width 0.2) (layer "F.Cu") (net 18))
 (segment (start 145.3642 106.5296) (end 143.8402 108.0536) (width 0.2) (layer "F.Cu") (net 19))
 (segment (start 143.8402 108.0536) (end 142.3574 108.0536) (width 0.2) (layer "F.Cu") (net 19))
 (segment (start 142.3574 108.0536) (end 141.351 109.06) (width 0.2) (layer "F.Cu") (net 19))
 (segment (start 143.8244 109.06) (end 145.0848 107.7996) (width 0.2) (layer "F.Cu") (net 20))
 (segment (start 143.351 109.06) (end 143.8244 109.06) (width 0.2) (layer "F.Cu") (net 20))
 (segment (start 145.0848 107.7996) (end 145.3642 107.7996) (width 0.2) (layer "F.Cu") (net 20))
 (segment (start 142.3508 110.0602) (end 141.351 111.06) (width 0.2) (layer "F.Cu") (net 21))
 (segment (start 145.3642 109.0696) (end 145.0848 109.0696) (width 0.2) (layer "F.Cu") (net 21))
 (segment (start 145.0848 109.0696) (end 144.0942 110.0602) (width 0.2) (layer "F.Cu") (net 21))
 (segment (start 144.0942 110.0602) (end 142.3508 110.0602) (width 0.2) (layer "F.Cu") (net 21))
 (segment (start 144.3644 111.06) (end 145.0848 110.3396) (width 0.2) (layer "F.Cu") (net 22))
 (segment (start 143.351 111.06) (end 144.3644 111.06) (width 0.2) (layer "F.Cu") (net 22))
 (segment (start 145.0848 110.3396) (end 145.3642 110.3396) (width 0.2) (layer "F.Cu") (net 22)))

